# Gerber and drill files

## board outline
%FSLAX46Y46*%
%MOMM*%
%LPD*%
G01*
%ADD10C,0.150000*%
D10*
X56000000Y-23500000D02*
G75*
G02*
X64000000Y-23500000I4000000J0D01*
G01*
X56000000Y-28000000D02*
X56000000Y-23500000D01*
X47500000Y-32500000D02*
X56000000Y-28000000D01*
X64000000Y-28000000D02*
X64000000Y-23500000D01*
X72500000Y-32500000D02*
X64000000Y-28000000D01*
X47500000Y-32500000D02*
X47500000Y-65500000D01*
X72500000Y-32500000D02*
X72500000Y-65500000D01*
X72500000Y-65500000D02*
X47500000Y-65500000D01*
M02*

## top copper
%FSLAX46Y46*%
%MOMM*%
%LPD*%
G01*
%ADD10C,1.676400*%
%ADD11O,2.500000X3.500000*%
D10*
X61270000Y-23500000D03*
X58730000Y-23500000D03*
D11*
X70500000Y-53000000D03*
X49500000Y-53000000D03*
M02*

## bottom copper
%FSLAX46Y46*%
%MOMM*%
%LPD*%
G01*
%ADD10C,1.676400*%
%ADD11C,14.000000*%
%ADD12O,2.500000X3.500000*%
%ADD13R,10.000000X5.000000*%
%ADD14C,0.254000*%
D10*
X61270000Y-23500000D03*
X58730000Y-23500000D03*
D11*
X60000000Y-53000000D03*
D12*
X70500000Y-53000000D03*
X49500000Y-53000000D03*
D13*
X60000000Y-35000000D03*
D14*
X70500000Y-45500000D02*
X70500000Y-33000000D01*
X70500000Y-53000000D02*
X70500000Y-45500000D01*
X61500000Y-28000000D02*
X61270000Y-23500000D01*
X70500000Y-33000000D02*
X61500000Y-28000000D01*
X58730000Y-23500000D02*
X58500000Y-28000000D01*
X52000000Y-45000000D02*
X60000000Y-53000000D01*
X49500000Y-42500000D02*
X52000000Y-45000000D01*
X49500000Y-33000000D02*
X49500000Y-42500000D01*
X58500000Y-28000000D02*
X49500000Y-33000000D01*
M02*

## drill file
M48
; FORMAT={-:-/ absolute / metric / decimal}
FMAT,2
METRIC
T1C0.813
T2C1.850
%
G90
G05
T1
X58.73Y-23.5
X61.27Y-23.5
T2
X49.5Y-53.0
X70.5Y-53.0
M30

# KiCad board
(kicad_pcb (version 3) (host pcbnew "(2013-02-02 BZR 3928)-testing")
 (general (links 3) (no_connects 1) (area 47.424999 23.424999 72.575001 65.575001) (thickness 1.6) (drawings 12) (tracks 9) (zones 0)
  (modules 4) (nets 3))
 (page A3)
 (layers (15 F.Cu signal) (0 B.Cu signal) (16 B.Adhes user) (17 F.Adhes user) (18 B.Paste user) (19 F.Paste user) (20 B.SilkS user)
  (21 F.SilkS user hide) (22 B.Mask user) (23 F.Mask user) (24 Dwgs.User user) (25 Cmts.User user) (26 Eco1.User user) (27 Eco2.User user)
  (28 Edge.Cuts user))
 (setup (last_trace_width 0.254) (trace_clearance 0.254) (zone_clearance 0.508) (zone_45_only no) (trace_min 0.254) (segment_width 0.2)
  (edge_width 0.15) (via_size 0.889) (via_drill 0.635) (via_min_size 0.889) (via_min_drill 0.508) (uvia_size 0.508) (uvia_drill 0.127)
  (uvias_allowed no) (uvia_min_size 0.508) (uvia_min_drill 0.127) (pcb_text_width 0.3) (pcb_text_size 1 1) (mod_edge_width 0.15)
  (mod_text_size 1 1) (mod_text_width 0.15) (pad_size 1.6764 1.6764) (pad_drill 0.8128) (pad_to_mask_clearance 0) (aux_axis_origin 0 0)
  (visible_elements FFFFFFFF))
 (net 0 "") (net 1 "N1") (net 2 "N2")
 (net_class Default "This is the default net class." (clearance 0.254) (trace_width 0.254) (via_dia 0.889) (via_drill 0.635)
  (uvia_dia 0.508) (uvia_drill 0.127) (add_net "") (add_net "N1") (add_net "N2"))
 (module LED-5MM (layer F.Cu) (at 60 23.5 180)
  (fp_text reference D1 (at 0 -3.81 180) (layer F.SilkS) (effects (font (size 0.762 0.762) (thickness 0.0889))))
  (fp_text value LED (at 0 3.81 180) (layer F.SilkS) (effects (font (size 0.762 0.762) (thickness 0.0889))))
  (pad 1 thru_hole circle (at -1.27 0 180) (size 1.6764 1.6764) (drill 0.8128) (layers *.Cu *.Mask) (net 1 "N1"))
  (pad 2 thru_hole circle (at 1.27 0 180) (size 1.6764 1.6764) (drill 0.8128) (layers *.Cu *.Mask) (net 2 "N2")))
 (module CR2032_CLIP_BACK (layer F.Cu) (at 60 53 180)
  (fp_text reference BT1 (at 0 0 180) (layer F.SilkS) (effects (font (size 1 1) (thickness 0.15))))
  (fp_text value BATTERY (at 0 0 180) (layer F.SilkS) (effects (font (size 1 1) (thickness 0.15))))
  (pad 2 smd circle (at 0 0 180) (size 14 14) (layers B.Cu B.Mask) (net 2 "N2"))
  (pad 1 thru_hole oval (at -10.5 0 180) (size 2.5 3.5) (drill 1.85) (layers *.Cu *.Mask F.SilkS) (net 1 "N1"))
  (pad 1 thru_hole oval (at 10.5 0 180) (size 2.5 3.5) (drill 1.85) (layers *.Cu *.Mask F.SilkS) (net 1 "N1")))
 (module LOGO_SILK (layer F.Cu) (at 60 45)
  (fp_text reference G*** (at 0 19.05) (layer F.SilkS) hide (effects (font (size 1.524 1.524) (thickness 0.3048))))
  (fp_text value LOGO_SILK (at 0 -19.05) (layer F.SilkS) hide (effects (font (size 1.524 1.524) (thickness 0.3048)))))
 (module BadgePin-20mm (layer F.Cu) (at 60 35)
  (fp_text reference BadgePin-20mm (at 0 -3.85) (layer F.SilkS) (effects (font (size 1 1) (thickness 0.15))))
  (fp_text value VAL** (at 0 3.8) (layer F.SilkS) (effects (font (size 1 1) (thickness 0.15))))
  (pad 1 smd rect (at 0 0) (size 10 5) (layers B.Cu B.Mask)))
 (gr_arc (start 60 23.5) (end 56 23.5) (angle 180) (layer Edge.Cuts) (width 0.15))
 (gr_line (start 56 28) (end 56 23.5) (angle 90) (layer Edge.Cuts) (width 0.15))
 (gr_line (start 47.5 32.5) (end 56 28) (angle 90) (layer Edge.Cuts) (width 0.15))
 (gr_line (start 64 28) (end 64 23.5) (angle 90) (layer Edge.Cuts) (width 0.15))
 (gr_line (start 72.5 32.5) (end 64 28) (angle 90) (layer Edge.Cuts) (width 0.15))
 (gr_line (start 47.5 32.5) (end 47.5 65.5) (angle 90) (layer Edge.Cuts) (width 0.15))
 (gr_line (start 72.5 32.5) (end 72.5 65.5) (angle 90) (layer Edge.Cuts) (width 0.15))
 (gr_line (start 72.5 65.5) (end 47.5 65.5) (angle 90) (layer Edge.Cuts) (width 0.15))
 (segment (start 70.5 45.5) (end 70.5 33) (width 0.254) (layer B.Cu) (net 1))
 (segment (start 70.5 53) (end 70.5 45.5) (width 0.254) (layer B.Cu) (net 1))
 (segment (start 61.5 28) (end 61.27 23.5) (width 0.254) (layer B.Cu) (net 1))
 (segment (start 70.5 33) (end 61.5 28) (width 0.254) (layer B.Cu) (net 1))
 (segment (start 58.73 23.5) (end 58.5 28) (width 0.254) (layer B.Cu) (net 2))
 (segment (start 52 45) (end 60 53) (width 0.254) (layer B.Cu) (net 2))
 (segment (start 49.5 42.5) (end 52 45) (width 0.254) (layer B.Cu) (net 2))
 (segment (start 49.5 33) (end 49.5 42.5) (width 0.254) (layer B.Cu) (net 2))
 (segment (start 58.5 28) (end 49.5 33) (width 0.254) (layer B.Cu) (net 2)))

